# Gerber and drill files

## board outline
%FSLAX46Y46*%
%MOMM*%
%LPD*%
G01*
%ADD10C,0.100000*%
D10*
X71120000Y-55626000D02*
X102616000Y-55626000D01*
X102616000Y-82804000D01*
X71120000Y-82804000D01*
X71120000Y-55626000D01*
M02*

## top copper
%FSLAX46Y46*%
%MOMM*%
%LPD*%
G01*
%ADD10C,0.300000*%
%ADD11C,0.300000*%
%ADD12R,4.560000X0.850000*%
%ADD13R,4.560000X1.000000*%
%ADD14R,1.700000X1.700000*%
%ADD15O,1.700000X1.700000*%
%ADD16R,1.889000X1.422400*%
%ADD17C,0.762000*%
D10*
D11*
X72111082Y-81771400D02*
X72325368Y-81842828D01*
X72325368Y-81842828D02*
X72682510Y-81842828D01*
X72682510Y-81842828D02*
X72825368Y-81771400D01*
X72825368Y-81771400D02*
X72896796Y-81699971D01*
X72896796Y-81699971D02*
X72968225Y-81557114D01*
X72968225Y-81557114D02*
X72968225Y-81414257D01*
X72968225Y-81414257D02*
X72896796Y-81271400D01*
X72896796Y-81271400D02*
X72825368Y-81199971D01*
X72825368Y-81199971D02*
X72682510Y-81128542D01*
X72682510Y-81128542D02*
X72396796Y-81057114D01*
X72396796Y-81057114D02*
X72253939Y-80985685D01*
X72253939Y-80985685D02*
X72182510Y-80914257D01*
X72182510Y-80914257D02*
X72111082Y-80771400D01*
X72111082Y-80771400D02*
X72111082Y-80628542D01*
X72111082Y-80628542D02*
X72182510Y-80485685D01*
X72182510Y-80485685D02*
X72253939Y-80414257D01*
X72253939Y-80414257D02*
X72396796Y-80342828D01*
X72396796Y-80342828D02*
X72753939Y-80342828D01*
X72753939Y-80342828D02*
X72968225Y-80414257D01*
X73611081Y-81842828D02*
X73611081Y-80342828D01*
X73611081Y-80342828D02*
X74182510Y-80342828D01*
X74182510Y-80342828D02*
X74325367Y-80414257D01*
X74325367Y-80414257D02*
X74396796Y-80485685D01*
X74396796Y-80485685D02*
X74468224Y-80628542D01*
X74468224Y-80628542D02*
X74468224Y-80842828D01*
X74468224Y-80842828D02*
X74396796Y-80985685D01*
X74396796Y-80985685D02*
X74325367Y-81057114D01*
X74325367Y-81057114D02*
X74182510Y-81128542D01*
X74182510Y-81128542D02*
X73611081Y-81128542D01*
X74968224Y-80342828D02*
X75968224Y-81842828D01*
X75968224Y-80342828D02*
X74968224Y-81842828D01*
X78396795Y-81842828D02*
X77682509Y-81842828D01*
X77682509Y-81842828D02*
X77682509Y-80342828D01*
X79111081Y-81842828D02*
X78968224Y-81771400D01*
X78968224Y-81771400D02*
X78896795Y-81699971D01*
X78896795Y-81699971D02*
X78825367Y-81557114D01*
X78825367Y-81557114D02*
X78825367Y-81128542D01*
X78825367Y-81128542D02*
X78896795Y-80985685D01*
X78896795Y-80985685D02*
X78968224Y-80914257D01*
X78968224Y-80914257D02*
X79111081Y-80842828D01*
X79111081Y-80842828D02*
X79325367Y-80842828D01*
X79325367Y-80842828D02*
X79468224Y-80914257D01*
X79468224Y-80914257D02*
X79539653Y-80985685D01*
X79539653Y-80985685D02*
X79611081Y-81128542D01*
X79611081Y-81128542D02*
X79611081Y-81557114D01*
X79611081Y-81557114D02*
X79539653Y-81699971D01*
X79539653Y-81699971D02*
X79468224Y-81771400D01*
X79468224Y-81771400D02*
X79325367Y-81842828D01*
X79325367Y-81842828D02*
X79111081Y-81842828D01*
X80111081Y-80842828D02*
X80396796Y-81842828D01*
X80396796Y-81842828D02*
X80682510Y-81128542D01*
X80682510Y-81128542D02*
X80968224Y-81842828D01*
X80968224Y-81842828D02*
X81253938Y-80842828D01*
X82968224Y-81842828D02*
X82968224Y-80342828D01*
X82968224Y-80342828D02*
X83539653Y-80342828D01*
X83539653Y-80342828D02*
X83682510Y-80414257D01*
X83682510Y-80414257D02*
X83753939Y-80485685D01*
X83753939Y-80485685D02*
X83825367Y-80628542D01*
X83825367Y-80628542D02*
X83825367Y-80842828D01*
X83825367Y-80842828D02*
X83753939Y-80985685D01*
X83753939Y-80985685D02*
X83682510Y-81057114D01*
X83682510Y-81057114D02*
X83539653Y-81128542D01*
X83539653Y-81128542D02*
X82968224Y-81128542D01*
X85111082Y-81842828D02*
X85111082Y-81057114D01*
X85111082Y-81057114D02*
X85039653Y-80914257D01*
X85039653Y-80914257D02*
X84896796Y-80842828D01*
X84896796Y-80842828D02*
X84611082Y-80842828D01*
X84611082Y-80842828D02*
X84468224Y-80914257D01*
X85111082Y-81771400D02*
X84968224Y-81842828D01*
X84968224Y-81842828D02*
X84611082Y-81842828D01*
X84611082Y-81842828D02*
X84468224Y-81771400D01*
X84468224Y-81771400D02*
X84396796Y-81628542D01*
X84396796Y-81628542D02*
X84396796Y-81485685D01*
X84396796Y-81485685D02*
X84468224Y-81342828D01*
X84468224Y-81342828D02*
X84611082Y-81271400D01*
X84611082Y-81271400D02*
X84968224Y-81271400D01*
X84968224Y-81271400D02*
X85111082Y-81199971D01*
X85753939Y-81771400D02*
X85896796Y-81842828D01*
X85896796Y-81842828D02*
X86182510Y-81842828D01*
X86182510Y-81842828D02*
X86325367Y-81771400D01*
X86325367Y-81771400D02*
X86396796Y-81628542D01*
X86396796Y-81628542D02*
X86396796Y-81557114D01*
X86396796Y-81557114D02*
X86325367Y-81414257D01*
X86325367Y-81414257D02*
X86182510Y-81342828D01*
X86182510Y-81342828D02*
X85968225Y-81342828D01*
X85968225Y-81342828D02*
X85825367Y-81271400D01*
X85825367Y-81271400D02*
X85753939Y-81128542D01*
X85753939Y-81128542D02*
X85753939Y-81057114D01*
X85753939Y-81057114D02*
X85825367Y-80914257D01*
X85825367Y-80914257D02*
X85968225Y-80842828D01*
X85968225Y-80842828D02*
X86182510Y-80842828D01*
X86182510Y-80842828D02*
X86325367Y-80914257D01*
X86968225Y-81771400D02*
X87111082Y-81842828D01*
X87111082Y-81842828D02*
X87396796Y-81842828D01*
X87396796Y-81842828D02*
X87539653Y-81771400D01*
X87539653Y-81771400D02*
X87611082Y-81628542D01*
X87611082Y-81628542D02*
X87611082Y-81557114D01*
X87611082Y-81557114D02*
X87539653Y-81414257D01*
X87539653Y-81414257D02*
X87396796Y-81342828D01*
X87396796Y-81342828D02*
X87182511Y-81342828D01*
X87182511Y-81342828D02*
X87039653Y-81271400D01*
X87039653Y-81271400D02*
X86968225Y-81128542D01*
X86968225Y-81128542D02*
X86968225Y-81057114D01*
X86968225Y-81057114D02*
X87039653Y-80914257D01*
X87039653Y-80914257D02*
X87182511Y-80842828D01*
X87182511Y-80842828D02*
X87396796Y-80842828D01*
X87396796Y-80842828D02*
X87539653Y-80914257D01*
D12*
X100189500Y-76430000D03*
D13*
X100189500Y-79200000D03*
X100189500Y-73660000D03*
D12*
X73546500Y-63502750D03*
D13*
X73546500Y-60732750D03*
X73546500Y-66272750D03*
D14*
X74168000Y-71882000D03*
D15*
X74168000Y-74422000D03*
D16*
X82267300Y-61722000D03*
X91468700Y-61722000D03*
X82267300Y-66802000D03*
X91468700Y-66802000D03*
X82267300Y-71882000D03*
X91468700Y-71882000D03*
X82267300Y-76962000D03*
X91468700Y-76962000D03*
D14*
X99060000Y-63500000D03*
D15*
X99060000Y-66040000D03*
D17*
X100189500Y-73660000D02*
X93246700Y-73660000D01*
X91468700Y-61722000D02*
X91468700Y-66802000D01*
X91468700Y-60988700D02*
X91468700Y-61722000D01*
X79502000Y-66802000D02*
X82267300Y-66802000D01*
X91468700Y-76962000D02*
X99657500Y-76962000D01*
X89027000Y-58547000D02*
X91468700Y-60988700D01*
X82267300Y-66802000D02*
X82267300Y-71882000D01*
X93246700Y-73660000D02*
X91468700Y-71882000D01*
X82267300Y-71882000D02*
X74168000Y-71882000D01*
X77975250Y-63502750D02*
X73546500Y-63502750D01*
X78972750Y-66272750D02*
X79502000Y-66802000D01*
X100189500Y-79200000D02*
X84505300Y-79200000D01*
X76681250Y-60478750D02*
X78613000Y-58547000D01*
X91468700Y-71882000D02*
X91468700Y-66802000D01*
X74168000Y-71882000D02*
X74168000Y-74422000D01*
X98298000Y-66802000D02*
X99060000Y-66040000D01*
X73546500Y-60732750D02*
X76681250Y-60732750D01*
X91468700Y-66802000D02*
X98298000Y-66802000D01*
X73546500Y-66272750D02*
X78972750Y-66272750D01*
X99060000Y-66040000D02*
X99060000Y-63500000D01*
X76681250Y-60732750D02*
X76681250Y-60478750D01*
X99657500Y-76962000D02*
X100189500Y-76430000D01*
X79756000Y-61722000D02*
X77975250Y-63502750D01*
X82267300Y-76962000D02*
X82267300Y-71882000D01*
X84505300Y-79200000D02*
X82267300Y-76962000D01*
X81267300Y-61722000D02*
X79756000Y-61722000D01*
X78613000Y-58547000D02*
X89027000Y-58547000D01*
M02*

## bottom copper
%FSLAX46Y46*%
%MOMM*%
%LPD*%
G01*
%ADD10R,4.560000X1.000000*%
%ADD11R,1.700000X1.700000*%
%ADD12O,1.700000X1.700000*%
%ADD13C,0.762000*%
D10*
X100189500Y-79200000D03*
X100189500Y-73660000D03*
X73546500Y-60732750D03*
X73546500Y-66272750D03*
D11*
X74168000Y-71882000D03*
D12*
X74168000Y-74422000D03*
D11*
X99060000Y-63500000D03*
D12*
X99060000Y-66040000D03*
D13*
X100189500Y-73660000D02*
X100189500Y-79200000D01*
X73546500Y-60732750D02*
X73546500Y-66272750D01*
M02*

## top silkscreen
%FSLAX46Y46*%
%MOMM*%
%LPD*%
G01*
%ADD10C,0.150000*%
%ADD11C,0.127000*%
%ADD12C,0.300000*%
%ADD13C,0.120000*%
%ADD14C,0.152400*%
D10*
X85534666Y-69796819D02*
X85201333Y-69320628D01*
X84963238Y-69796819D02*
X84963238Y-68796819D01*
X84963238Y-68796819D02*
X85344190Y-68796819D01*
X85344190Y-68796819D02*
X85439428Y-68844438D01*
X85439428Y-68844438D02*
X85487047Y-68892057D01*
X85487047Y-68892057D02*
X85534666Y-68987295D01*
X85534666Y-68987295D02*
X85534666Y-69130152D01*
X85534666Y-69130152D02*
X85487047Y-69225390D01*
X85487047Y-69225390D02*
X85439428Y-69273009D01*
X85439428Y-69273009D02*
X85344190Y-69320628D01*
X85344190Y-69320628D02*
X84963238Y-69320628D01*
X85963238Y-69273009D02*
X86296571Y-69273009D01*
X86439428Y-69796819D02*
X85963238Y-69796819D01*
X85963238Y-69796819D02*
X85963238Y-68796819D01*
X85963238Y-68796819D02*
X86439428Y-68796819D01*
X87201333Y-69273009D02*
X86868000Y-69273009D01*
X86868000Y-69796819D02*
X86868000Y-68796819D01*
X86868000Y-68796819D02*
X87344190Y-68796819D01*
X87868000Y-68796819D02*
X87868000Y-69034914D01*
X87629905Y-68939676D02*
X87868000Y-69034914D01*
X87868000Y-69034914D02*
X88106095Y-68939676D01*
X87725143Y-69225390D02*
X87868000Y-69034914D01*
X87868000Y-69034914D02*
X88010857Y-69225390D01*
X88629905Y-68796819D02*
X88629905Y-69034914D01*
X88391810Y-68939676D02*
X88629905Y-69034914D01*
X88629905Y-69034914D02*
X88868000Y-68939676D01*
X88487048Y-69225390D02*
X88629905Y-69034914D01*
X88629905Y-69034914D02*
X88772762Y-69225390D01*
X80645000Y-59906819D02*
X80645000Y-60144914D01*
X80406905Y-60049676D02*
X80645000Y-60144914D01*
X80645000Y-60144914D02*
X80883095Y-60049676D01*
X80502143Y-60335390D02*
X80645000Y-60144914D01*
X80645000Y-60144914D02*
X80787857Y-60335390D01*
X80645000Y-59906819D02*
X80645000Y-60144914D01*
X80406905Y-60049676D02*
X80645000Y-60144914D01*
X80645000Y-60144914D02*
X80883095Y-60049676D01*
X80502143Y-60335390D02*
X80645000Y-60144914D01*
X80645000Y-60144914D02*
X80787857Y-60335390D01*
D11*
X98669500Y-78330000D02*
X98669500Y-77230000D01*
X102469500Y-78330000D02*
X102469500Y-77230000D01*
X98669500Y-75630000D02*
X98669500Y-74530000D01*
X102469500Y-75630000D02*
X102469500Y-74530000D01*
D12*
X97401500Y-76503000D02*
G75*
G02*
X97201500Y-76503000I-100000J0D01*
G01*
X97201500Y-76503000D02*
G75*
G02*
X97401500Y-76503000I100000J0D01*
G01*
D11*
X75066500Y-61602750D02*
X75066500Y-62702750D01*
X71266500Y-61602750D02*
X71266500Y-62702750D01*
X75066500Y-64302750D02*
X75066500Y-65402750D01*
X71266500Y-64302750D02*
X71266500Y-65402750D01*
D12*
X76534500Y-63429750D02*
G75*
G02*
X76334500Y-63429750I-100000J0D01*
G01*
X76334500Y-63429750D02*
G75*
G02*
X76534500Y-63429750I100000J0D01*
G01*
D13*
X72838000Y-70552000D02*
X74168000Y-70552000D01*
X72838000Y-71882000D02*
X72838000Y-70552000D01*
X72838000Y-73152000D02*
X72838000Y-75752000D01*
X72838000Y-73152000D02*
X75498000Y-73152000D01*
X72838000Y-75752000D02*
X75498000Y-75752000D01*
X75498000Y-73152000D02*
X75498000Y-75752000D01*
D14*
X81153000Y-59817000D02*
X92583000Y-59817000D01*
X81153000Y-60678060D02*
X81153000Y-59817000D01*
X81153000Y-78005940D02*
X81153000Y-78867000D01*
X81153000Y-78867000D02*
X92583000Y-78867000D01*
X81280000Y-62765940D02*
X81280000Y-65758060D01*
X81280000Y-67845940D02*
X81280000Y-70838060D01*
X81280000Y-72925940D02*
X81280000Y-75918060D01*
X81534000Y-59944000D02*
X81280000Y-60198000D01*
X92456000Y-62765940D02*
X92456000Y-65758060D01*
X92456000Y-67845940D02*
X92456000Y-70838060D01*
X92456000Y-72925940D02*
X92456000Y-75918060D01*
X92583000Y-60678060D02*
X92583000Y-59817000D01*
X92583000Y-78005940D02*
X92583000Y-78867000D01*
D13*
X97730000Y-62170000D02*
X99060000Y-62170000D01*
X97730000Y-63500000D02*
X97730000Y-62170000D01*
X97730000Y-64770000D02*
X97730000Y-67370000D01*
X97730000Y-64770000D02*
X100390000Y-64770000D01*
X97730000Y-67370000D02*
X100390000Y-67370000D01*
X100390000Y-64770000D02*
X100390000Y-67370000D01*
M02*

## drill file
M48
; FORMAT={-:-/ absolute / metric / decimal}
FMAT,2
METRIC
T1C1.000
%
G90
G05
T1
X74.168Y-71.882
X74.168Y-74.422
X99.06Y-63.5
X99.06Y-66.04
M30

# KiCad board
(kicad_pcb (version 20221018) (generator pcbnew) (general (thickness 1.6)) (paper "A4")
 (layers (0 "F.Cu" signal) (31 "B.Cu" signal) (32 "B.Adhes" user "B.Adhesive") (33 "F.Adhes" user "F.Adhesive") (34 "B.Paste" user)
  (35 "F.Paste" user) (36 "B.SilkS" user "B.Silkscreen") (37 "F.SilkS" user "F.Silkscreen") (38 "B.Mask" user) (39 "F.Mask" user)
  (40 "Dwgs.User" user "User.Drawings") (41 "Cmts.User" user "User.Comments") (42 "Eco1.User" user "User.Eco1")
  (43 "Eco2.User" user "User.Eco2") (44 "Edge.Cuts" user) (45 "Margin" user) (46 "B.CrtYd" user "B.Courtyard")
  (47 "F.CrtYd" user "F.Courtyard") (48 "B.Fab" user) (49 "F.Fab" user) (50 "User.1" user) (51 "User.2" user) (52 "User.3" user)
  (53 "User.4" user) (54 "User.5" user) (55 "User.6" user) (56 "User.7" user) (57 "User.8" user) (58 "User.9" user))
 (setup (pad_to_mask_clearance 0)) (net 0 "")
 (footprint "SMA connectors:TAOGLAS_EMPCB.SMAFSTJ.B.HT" (layer "F.Cu") (at 100.1895 76.43 90)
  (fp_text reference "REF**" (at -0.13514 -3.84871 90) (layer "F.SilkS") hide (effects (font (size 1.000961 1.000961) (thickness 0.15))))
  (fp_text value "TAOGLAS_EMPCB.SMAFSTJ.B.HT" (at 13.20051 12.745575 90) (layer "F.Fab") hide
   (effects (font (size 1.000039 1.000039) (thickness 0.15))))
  (fp_line (start -1.9 -1.52) (end -0.8 -1.52) (stroke (width 0.127) (type solid)) (layer "F.SilkS"))
  (fp_line (start -1.9 2.28) (end -0.8 2.28) (stroke (width 0.127) (type solid)) (layer "F.SilkS"))
  (fp_line (start 0.8 -1.52) (end 1.9 -1.52) (stroke (width 0.127) (type solid)) (layer "F.SilkS"))
  (fp_line (start 0.8 2.28) (end 1.9 2.28) (stroke (width 0.127) (type solid)) (layer "F.SilkS"))
  (fp_circle (center -0.073 -2.888) (end 0.027 -2.888) (stroke (width 0.3) (type solid)) (fill none) (layer "F.SilkS"))
  (pad "1" smd rect (at 0 0 90) (size 0.85 4.56) (layers "F.Cu" "F.Paste" "F.Mask") (solder_mask_margin 0.102))
  (pad "SH1" smd rect (at -2.77 0 90) (size 1 4.56) (layers "F.Cu" "F.Paste" "F.Mask") (solder_mask_margin 0.102))
  (pad "SH2" smd rect (at 2.77 0 90) (size 1 4.56) (layers "F.Cu" "F.Paste" "F.Mask") (solder_mask_margin 0.102))
  (pad "SH3" smd rect (at -2.77 0 90) (size 1 4.56) (layers "B.Cu" "B.Paste" "B.Mask") (solder_mask_margin 0.102))
  (pad "SH4" smd rect (at 2.77 0 90) (size 1 4.56) (layers "B.Cu" "B.Paste" "B.Mask") (solder_mask_margin 0.102)))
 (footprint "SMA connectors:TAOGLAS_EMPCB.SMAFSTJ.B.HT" (layer "F.Cu") (at 73.5465 63.50275 -90)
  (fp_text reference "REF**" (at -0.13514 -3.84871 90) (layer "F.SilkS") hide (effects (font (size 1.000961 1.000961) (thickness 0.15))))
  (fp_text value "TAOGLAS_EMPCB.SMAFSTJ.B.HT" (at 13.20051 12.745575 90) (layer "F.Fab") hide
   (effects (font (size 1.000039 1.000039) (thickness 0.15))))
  (fp_line (start -1.9 -1.52) (end -0.8 -1.52) (stroke (width 0.127) (type solid)) (layer "F.SilkS"))
  (fp_line (start -1.9 2.28) (end -0.8 2.28) (stroke (width 0.127) (type solid)) (layer "F.SilkS"))
  (fp_line (start 0.8 -1.52) (end 1.9 -1.52) (stroke (width 0.127) (type solid)) (layer "F.SilkS"))
  (fp_line (start 0.8 2.28) (end 1.9 2.28) (stroke (width 0.127) (type solid)) (layer "F.SilkS"))
  (fp_circle (center -0.073 -2.888) (end 0.027 -2.888) (stroke (width 0.3) (type solid)) (fill none) (layer "F.SilkS"))
  (pad "1" smd rect (at 0 0 270) (size 0.85 4.56) (layers "F.Cu" "F.Paste" "F.Mask") (solder_mask_margin 0.102))
  (pad "SH1" smd rect (at -2.77 0 270) (size 1 4.56) (layers "F.Cu" "F.Paste" "F.Mask") (solder_mask_margin 0.102))
  (pad "SH2" smd rect (at 2.77 0 270) (size 1 4.56) (layers "F.Cu" "F.Paste" "F.Mask") (solder_mask_margin 0.102))
  (pad "SH3" smd rect (at -2.77 0 270) (size 1 4.56) (layers "B.Cu" "B.Paste" "B.Mask") (solder_mask_margin 0.102))
  (pad "SH4" smd rect (at 2.77 0 270) (size 1 4.56) (layers "B.Cu" "B.Paste" "B.Mask") (solder_mask_margin 0.102)))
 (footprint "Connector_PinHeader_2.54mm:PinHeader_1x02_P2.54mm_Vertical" (layer "F.Cu") (at 74.168 71.882)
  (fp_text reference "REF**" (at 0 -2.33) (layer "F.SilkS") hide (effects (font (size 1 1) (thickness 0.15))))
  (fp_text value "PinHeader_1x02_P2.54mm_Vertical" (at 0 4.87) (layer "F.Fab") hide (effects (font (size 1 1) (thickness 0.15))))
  (fp_line (start -1.33 -1.33) (end 0 -1.33) (stroke (width 0.12) (type solid)) (layer "F.SilkS"))
  (fp_line (start -1.33 0) (end -1.33 -1.33) (stroke (width 0.12) (type solid)) (layer "F.SilkS"))
  (fp_line (start -1.33 1.27) (end -1.33 3.87) (stroke (width 0.12) (type solid)) (layer "F.SilkS"))
  (fp_line (start -1.33 1.27) (end 1.33 1.27) (stroke (width 0.12) (type solid)) (layer "F.SilkS"))
  (fp_line (start -1.33 3.87) (end 1.33 3.87) (stroke (width 0.12) (type solid)) (layer "F.SilkS"))
  (fp_line (start 1.33 1.27) (end 1.33 3.87) (stroke (width 0.12) (type solid)) (layer "F.SilkS"))
  (pad "1" thru_hole rect (at 0 0) (size 1.7 1.7) (drill 1) (layers "*.Cu" "*.Mask"))
  (pad "2" thru_hole oval (at 0 2.54) (size 1.7 1.7) (drill 1) (layers "*.Cu" "*.Mask")))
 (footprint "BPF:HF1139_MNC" (layer "F.Cu") (at 86.868 69.342)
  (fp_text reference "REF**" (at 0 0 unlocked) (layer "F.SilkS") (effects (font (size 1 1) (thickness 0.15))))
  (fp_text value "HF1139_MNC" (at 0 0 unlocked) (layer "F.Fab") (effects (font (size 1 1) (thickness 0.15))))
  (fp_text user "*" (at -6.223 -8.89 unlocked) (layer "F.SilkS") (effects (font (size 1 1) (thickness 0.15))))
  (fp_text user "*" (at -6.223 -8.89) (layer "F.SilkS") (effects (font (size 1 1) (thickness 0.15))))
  (fp_line (start -5.715 -9.525) (end 5.715 -9.525) (stroke (width 0.1524) (type solid)) (layer "F.SilkS"))
  (fp_line (start -5.715 -8.66394) (end -5.715 -9.525) (stroke (width 0.1524) (type solid)) (layer "F.SilkS"))
  (fp_line (start -5.715 8.66394) (end -5.715 9.525) (stroke (width 0.1524) (type solid)) (layer "F.SilkS"))
  (fp_line (start -5.715 9.525) (end 5.715 9.525) (stroke (width 0.1524) (type solid)) (layer "F.SilkS"))
  (fp_line (start -5.588 -6.57606) (end -5.588 -3.58394) (stroke (width 0.1524) (type solid)) (layer "F.SilkS"))
  (fp_line (start -5.588 -1.49606) (end -5.588 1.49606) (stroke (width 0.1524) (type solid)) (layer "F.SilkS"))
  (fp_line (start -5.588 3.58394) (end -5.588 6.57606) (stroke (width 0.1524) (type solid)) (layer "F.SilkS"))
  (fp_line (start -5.334 -9.398) (end -5.588 -9.144) (stroke (width 0.1524) (type solid)) (layer "F.SilkS"))
  (fp_line (start 5.588 -6.57606) (end 5.588 -3.58394) (stroke (width 0.1524) (type solid)) (layer "F.SilkS"))
  (fp_line (start 5.588 -1.49606) (end 5.588 1.49606) (stroke (width 0.1524) (type solid)) (layer "F.SilkS"))
  (fp_line (start 5.588 3.58394) (end 5.588 6.57606) (stroke (width 0.1524) (type solid)) (layer "F.SilkS"))
  (fp_line (start 5.715 -8.66394) (end 5.715 -9.525) (stroke (width 0.1524) (type solid)) (layer "F.SilkS"))
  (fp_line (start 5.715 8.66394) (end 5.715 9.525) (stroke (width 0.1524) (type solid)) (layer "F.SilkS"))
  (pad "1" smd rect (at -4.6007 -7.62) (size 1.889 1.4224) (layers "F.Cu" "F.Paste" "F.Mask"))
  (pad "2" smd rect (at 4.6007 -7.62) (size 1.889 1.4224) (layers "F.Cu" "F.Paste" "F.Mask"))
  (pad "3" smd rect (at -4.6007 -2.54) (size 1.889 1.4224) (layers "F.Cu" "F.Paste" "F.Mask"))
  (pad "4" smd rect (at 4.6007 -2.54) (size 1.889 1.4224) (layers "F.Cu" "F.Paste" "F.Mask"))
  (pad "5" smd rect (at -4.6007 2.54) (size 1.889 1.4224) (layers "F.Cu" "F.Paste" "F.Mask"))
  (pad "6" smd rect (at 4.6007 2.54) (size 1.889 1.4224) (layers "F.Cu" "F.Paste" "F.Mask"))
  (pad "7" smd rect (at -4.6007 7.62) (size 1.889 1.4224) (layers "F.Cu" "F.Paste" "F.Mask"))
  (pad "8" smd rect (at 4.6007 7.62) (size 1.889 1.4224) (layers "F.Cu" "F.Paste" "F.Mask")))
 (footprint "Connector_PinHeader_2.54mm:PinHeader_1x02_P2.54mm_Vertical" (layer "F.Cu") (at 99.06 63.5)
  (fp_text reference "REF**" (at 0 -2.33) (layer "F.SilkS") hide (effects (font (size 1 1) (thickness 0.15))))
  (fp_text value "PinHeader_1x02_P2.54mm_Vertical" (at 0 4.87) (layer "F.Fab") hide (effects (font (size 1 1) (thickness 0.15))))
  (fp_line (start -1.33 -1.33) (end 0 -1.33) (stroke (width 0.12) (type solid)) (layer "F.SilkS"))
  (fp_line (start -1.33 0) (end -1.33 -1.33) (stroke (width 0.12) (type solid)) (layer "F.SilkS"))
  (fp_line (start -1.33 1.27) (end -1.33 3.87) (stroke (width 0.12) (type solid)) (layer "F.SilkS"))
  (fp_line (start -1.33 1.27) (end 1.33 1.27) (stroke (width 0.12) (type solid)) (layer "F.SilkS"))
  (fp_line (start -1.33 3.87) (end 1.33 3.87) (stroke (width 0.12) (type solid)) (layer "F.SilkS"))
  (fp_line (start 1.33 1.27) (end 1.33 3.87) (stroke (width 0.12) (type solid)) (layer "F.SilkS"))
  (pad "1" thru_hole rect (at 0 0) (size 1.7 1.7) (drill 1) (layers "*.Cu" "*.Mask"))
  (pad "2" thru_hole oval (at 0 2.54) (size 1.7 1.7) (drill 1) (layers "*.Cu" "*.Mask")))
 (gr_rect (start 71.12 55.626) (end 102.616 82.804) (stroke (width 0.1) (type default)) (fill none) (layer "Edge.Cuts"))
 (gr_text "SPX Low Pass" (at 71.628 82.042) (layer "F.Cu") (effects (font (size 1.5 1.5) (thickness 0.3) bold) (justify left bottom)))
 (segment (start 100.1895 73.66) (end 93.2467 73.66) (width 0.762) (layer "F.Cu") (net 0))
 (segment (start 91.4687 61.722) (end 91.4687 66.802) (width 0.762) (layer "F.Cu") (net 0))
 (segment (start 91.4687 60.9887) (end 91.4687 61.722) (width 0.762) (layer "F.Cu") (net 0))
 (segment (start 79.502 66.802) (end 82.2673 66.802) (width 0.762) (layer "F.Cu") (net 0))
 (segment (start 91.4687 76.962) (end 99.6575 76.962) (width 0.762) (layer "F.Cu") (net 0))
 (segment (start 89.027 58.547) (end 91.4687 60.9887) (width 0.762) (layer "F.Cu") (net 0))
 (segment (start 82.2673 66.802) (end 82.2673 71.882) (width 0.762) (layer "F.Cu") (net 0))
 (segment (start 93.2467 73.66) (end 91.4687 71.882) (width 0.762) (layer "F.Cu") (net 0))
 (segment (start 82.2673 71.882) (end 74.168 71.882) (width 0.762) (layer "F.Cu") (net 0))
 (segment (start 77.97525 63.50275) (end 73.5465 63.50275) (width 0.762) (layer "F.Cu") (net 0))
 (segment (start 78.97275 66.27275) (end 79.502 66.802) (width 0.762) (layer "F.Cu") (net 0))
 (segment (start 100.1895 79.2) (end 84.5053 79.2) (width 0.762) (layer "F.Cu") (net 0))
 (segment (start 76.68125 60.47875) (end 78.613 58.547) (width 0.762) (layer "F.Cu") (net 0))
 (segment (start 91.4687 71.882) (end 91.4687 66.802) (width 0.762) (layer "F.Cu") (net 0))
 (segment (start 74.168 71.882) (end 74.168 74.422) (width 0.762) (layer "F.Cu") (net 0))
 (segment (start 98.298 66.802) (end 99.06 66.04) (width 0.762) (layer "F.Cu") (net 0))
 (segment (start 73.5465 60.73275) (end 76.68125 60.73275) (width 0.762) (layer "F.Cu") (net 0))
 (segment (start 91.4687 66.802) (end 98.298 66.802) (width 0.762) (layer "F.Cu") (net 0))
 (segment (start 73.5465 66.27275) (end 78.97275 66.27275) (width 0.762) (layer "F.Cu") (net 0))
 (segment (start 99.06 66.04) (end 99.06 63.5) (width 0.762) (layer "F.Cu") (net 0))
 (segment (start 76.68125 60.73275) (end 76.68125 60.47875) (width 0.762) (layer "F.Cu") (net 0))
 (segment (start 99.6575 76.962) (end 100.1895 76.43) (width 0.762) (layer "F.Cu") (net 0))
 (segment (start 79.756 61.722) (end 77.97525 63.50275) (width 0.762) (layer "F.Cu") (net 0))
 (segment (start 82.2673 76.962) (end 82.2673 71.882) (width 0.762) (layer "F.Cu") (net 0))
 (segment (start 84.5053 79.2) (end 82.2673 76.962) (width 0.762) (layer "F.Cu") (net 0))
 (segment (start 81.2673 61.722) (end 79.756 61.722) (width 0.762) (layer "F.Cu") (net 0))
 (segment (start 78.613 58.547) (end 89.027 58.547) (width 0.762) (layer "F.Cu") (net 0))
 (segment (start 100.1895 73.66) (end 100.1895 79.2) (width 0.762) (layer "B.Cu") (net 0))
 (segment (start 73.5465 60.73275) (end 73.5465 66.27275) (width 0.762) (layer "B.Cu") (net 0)))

